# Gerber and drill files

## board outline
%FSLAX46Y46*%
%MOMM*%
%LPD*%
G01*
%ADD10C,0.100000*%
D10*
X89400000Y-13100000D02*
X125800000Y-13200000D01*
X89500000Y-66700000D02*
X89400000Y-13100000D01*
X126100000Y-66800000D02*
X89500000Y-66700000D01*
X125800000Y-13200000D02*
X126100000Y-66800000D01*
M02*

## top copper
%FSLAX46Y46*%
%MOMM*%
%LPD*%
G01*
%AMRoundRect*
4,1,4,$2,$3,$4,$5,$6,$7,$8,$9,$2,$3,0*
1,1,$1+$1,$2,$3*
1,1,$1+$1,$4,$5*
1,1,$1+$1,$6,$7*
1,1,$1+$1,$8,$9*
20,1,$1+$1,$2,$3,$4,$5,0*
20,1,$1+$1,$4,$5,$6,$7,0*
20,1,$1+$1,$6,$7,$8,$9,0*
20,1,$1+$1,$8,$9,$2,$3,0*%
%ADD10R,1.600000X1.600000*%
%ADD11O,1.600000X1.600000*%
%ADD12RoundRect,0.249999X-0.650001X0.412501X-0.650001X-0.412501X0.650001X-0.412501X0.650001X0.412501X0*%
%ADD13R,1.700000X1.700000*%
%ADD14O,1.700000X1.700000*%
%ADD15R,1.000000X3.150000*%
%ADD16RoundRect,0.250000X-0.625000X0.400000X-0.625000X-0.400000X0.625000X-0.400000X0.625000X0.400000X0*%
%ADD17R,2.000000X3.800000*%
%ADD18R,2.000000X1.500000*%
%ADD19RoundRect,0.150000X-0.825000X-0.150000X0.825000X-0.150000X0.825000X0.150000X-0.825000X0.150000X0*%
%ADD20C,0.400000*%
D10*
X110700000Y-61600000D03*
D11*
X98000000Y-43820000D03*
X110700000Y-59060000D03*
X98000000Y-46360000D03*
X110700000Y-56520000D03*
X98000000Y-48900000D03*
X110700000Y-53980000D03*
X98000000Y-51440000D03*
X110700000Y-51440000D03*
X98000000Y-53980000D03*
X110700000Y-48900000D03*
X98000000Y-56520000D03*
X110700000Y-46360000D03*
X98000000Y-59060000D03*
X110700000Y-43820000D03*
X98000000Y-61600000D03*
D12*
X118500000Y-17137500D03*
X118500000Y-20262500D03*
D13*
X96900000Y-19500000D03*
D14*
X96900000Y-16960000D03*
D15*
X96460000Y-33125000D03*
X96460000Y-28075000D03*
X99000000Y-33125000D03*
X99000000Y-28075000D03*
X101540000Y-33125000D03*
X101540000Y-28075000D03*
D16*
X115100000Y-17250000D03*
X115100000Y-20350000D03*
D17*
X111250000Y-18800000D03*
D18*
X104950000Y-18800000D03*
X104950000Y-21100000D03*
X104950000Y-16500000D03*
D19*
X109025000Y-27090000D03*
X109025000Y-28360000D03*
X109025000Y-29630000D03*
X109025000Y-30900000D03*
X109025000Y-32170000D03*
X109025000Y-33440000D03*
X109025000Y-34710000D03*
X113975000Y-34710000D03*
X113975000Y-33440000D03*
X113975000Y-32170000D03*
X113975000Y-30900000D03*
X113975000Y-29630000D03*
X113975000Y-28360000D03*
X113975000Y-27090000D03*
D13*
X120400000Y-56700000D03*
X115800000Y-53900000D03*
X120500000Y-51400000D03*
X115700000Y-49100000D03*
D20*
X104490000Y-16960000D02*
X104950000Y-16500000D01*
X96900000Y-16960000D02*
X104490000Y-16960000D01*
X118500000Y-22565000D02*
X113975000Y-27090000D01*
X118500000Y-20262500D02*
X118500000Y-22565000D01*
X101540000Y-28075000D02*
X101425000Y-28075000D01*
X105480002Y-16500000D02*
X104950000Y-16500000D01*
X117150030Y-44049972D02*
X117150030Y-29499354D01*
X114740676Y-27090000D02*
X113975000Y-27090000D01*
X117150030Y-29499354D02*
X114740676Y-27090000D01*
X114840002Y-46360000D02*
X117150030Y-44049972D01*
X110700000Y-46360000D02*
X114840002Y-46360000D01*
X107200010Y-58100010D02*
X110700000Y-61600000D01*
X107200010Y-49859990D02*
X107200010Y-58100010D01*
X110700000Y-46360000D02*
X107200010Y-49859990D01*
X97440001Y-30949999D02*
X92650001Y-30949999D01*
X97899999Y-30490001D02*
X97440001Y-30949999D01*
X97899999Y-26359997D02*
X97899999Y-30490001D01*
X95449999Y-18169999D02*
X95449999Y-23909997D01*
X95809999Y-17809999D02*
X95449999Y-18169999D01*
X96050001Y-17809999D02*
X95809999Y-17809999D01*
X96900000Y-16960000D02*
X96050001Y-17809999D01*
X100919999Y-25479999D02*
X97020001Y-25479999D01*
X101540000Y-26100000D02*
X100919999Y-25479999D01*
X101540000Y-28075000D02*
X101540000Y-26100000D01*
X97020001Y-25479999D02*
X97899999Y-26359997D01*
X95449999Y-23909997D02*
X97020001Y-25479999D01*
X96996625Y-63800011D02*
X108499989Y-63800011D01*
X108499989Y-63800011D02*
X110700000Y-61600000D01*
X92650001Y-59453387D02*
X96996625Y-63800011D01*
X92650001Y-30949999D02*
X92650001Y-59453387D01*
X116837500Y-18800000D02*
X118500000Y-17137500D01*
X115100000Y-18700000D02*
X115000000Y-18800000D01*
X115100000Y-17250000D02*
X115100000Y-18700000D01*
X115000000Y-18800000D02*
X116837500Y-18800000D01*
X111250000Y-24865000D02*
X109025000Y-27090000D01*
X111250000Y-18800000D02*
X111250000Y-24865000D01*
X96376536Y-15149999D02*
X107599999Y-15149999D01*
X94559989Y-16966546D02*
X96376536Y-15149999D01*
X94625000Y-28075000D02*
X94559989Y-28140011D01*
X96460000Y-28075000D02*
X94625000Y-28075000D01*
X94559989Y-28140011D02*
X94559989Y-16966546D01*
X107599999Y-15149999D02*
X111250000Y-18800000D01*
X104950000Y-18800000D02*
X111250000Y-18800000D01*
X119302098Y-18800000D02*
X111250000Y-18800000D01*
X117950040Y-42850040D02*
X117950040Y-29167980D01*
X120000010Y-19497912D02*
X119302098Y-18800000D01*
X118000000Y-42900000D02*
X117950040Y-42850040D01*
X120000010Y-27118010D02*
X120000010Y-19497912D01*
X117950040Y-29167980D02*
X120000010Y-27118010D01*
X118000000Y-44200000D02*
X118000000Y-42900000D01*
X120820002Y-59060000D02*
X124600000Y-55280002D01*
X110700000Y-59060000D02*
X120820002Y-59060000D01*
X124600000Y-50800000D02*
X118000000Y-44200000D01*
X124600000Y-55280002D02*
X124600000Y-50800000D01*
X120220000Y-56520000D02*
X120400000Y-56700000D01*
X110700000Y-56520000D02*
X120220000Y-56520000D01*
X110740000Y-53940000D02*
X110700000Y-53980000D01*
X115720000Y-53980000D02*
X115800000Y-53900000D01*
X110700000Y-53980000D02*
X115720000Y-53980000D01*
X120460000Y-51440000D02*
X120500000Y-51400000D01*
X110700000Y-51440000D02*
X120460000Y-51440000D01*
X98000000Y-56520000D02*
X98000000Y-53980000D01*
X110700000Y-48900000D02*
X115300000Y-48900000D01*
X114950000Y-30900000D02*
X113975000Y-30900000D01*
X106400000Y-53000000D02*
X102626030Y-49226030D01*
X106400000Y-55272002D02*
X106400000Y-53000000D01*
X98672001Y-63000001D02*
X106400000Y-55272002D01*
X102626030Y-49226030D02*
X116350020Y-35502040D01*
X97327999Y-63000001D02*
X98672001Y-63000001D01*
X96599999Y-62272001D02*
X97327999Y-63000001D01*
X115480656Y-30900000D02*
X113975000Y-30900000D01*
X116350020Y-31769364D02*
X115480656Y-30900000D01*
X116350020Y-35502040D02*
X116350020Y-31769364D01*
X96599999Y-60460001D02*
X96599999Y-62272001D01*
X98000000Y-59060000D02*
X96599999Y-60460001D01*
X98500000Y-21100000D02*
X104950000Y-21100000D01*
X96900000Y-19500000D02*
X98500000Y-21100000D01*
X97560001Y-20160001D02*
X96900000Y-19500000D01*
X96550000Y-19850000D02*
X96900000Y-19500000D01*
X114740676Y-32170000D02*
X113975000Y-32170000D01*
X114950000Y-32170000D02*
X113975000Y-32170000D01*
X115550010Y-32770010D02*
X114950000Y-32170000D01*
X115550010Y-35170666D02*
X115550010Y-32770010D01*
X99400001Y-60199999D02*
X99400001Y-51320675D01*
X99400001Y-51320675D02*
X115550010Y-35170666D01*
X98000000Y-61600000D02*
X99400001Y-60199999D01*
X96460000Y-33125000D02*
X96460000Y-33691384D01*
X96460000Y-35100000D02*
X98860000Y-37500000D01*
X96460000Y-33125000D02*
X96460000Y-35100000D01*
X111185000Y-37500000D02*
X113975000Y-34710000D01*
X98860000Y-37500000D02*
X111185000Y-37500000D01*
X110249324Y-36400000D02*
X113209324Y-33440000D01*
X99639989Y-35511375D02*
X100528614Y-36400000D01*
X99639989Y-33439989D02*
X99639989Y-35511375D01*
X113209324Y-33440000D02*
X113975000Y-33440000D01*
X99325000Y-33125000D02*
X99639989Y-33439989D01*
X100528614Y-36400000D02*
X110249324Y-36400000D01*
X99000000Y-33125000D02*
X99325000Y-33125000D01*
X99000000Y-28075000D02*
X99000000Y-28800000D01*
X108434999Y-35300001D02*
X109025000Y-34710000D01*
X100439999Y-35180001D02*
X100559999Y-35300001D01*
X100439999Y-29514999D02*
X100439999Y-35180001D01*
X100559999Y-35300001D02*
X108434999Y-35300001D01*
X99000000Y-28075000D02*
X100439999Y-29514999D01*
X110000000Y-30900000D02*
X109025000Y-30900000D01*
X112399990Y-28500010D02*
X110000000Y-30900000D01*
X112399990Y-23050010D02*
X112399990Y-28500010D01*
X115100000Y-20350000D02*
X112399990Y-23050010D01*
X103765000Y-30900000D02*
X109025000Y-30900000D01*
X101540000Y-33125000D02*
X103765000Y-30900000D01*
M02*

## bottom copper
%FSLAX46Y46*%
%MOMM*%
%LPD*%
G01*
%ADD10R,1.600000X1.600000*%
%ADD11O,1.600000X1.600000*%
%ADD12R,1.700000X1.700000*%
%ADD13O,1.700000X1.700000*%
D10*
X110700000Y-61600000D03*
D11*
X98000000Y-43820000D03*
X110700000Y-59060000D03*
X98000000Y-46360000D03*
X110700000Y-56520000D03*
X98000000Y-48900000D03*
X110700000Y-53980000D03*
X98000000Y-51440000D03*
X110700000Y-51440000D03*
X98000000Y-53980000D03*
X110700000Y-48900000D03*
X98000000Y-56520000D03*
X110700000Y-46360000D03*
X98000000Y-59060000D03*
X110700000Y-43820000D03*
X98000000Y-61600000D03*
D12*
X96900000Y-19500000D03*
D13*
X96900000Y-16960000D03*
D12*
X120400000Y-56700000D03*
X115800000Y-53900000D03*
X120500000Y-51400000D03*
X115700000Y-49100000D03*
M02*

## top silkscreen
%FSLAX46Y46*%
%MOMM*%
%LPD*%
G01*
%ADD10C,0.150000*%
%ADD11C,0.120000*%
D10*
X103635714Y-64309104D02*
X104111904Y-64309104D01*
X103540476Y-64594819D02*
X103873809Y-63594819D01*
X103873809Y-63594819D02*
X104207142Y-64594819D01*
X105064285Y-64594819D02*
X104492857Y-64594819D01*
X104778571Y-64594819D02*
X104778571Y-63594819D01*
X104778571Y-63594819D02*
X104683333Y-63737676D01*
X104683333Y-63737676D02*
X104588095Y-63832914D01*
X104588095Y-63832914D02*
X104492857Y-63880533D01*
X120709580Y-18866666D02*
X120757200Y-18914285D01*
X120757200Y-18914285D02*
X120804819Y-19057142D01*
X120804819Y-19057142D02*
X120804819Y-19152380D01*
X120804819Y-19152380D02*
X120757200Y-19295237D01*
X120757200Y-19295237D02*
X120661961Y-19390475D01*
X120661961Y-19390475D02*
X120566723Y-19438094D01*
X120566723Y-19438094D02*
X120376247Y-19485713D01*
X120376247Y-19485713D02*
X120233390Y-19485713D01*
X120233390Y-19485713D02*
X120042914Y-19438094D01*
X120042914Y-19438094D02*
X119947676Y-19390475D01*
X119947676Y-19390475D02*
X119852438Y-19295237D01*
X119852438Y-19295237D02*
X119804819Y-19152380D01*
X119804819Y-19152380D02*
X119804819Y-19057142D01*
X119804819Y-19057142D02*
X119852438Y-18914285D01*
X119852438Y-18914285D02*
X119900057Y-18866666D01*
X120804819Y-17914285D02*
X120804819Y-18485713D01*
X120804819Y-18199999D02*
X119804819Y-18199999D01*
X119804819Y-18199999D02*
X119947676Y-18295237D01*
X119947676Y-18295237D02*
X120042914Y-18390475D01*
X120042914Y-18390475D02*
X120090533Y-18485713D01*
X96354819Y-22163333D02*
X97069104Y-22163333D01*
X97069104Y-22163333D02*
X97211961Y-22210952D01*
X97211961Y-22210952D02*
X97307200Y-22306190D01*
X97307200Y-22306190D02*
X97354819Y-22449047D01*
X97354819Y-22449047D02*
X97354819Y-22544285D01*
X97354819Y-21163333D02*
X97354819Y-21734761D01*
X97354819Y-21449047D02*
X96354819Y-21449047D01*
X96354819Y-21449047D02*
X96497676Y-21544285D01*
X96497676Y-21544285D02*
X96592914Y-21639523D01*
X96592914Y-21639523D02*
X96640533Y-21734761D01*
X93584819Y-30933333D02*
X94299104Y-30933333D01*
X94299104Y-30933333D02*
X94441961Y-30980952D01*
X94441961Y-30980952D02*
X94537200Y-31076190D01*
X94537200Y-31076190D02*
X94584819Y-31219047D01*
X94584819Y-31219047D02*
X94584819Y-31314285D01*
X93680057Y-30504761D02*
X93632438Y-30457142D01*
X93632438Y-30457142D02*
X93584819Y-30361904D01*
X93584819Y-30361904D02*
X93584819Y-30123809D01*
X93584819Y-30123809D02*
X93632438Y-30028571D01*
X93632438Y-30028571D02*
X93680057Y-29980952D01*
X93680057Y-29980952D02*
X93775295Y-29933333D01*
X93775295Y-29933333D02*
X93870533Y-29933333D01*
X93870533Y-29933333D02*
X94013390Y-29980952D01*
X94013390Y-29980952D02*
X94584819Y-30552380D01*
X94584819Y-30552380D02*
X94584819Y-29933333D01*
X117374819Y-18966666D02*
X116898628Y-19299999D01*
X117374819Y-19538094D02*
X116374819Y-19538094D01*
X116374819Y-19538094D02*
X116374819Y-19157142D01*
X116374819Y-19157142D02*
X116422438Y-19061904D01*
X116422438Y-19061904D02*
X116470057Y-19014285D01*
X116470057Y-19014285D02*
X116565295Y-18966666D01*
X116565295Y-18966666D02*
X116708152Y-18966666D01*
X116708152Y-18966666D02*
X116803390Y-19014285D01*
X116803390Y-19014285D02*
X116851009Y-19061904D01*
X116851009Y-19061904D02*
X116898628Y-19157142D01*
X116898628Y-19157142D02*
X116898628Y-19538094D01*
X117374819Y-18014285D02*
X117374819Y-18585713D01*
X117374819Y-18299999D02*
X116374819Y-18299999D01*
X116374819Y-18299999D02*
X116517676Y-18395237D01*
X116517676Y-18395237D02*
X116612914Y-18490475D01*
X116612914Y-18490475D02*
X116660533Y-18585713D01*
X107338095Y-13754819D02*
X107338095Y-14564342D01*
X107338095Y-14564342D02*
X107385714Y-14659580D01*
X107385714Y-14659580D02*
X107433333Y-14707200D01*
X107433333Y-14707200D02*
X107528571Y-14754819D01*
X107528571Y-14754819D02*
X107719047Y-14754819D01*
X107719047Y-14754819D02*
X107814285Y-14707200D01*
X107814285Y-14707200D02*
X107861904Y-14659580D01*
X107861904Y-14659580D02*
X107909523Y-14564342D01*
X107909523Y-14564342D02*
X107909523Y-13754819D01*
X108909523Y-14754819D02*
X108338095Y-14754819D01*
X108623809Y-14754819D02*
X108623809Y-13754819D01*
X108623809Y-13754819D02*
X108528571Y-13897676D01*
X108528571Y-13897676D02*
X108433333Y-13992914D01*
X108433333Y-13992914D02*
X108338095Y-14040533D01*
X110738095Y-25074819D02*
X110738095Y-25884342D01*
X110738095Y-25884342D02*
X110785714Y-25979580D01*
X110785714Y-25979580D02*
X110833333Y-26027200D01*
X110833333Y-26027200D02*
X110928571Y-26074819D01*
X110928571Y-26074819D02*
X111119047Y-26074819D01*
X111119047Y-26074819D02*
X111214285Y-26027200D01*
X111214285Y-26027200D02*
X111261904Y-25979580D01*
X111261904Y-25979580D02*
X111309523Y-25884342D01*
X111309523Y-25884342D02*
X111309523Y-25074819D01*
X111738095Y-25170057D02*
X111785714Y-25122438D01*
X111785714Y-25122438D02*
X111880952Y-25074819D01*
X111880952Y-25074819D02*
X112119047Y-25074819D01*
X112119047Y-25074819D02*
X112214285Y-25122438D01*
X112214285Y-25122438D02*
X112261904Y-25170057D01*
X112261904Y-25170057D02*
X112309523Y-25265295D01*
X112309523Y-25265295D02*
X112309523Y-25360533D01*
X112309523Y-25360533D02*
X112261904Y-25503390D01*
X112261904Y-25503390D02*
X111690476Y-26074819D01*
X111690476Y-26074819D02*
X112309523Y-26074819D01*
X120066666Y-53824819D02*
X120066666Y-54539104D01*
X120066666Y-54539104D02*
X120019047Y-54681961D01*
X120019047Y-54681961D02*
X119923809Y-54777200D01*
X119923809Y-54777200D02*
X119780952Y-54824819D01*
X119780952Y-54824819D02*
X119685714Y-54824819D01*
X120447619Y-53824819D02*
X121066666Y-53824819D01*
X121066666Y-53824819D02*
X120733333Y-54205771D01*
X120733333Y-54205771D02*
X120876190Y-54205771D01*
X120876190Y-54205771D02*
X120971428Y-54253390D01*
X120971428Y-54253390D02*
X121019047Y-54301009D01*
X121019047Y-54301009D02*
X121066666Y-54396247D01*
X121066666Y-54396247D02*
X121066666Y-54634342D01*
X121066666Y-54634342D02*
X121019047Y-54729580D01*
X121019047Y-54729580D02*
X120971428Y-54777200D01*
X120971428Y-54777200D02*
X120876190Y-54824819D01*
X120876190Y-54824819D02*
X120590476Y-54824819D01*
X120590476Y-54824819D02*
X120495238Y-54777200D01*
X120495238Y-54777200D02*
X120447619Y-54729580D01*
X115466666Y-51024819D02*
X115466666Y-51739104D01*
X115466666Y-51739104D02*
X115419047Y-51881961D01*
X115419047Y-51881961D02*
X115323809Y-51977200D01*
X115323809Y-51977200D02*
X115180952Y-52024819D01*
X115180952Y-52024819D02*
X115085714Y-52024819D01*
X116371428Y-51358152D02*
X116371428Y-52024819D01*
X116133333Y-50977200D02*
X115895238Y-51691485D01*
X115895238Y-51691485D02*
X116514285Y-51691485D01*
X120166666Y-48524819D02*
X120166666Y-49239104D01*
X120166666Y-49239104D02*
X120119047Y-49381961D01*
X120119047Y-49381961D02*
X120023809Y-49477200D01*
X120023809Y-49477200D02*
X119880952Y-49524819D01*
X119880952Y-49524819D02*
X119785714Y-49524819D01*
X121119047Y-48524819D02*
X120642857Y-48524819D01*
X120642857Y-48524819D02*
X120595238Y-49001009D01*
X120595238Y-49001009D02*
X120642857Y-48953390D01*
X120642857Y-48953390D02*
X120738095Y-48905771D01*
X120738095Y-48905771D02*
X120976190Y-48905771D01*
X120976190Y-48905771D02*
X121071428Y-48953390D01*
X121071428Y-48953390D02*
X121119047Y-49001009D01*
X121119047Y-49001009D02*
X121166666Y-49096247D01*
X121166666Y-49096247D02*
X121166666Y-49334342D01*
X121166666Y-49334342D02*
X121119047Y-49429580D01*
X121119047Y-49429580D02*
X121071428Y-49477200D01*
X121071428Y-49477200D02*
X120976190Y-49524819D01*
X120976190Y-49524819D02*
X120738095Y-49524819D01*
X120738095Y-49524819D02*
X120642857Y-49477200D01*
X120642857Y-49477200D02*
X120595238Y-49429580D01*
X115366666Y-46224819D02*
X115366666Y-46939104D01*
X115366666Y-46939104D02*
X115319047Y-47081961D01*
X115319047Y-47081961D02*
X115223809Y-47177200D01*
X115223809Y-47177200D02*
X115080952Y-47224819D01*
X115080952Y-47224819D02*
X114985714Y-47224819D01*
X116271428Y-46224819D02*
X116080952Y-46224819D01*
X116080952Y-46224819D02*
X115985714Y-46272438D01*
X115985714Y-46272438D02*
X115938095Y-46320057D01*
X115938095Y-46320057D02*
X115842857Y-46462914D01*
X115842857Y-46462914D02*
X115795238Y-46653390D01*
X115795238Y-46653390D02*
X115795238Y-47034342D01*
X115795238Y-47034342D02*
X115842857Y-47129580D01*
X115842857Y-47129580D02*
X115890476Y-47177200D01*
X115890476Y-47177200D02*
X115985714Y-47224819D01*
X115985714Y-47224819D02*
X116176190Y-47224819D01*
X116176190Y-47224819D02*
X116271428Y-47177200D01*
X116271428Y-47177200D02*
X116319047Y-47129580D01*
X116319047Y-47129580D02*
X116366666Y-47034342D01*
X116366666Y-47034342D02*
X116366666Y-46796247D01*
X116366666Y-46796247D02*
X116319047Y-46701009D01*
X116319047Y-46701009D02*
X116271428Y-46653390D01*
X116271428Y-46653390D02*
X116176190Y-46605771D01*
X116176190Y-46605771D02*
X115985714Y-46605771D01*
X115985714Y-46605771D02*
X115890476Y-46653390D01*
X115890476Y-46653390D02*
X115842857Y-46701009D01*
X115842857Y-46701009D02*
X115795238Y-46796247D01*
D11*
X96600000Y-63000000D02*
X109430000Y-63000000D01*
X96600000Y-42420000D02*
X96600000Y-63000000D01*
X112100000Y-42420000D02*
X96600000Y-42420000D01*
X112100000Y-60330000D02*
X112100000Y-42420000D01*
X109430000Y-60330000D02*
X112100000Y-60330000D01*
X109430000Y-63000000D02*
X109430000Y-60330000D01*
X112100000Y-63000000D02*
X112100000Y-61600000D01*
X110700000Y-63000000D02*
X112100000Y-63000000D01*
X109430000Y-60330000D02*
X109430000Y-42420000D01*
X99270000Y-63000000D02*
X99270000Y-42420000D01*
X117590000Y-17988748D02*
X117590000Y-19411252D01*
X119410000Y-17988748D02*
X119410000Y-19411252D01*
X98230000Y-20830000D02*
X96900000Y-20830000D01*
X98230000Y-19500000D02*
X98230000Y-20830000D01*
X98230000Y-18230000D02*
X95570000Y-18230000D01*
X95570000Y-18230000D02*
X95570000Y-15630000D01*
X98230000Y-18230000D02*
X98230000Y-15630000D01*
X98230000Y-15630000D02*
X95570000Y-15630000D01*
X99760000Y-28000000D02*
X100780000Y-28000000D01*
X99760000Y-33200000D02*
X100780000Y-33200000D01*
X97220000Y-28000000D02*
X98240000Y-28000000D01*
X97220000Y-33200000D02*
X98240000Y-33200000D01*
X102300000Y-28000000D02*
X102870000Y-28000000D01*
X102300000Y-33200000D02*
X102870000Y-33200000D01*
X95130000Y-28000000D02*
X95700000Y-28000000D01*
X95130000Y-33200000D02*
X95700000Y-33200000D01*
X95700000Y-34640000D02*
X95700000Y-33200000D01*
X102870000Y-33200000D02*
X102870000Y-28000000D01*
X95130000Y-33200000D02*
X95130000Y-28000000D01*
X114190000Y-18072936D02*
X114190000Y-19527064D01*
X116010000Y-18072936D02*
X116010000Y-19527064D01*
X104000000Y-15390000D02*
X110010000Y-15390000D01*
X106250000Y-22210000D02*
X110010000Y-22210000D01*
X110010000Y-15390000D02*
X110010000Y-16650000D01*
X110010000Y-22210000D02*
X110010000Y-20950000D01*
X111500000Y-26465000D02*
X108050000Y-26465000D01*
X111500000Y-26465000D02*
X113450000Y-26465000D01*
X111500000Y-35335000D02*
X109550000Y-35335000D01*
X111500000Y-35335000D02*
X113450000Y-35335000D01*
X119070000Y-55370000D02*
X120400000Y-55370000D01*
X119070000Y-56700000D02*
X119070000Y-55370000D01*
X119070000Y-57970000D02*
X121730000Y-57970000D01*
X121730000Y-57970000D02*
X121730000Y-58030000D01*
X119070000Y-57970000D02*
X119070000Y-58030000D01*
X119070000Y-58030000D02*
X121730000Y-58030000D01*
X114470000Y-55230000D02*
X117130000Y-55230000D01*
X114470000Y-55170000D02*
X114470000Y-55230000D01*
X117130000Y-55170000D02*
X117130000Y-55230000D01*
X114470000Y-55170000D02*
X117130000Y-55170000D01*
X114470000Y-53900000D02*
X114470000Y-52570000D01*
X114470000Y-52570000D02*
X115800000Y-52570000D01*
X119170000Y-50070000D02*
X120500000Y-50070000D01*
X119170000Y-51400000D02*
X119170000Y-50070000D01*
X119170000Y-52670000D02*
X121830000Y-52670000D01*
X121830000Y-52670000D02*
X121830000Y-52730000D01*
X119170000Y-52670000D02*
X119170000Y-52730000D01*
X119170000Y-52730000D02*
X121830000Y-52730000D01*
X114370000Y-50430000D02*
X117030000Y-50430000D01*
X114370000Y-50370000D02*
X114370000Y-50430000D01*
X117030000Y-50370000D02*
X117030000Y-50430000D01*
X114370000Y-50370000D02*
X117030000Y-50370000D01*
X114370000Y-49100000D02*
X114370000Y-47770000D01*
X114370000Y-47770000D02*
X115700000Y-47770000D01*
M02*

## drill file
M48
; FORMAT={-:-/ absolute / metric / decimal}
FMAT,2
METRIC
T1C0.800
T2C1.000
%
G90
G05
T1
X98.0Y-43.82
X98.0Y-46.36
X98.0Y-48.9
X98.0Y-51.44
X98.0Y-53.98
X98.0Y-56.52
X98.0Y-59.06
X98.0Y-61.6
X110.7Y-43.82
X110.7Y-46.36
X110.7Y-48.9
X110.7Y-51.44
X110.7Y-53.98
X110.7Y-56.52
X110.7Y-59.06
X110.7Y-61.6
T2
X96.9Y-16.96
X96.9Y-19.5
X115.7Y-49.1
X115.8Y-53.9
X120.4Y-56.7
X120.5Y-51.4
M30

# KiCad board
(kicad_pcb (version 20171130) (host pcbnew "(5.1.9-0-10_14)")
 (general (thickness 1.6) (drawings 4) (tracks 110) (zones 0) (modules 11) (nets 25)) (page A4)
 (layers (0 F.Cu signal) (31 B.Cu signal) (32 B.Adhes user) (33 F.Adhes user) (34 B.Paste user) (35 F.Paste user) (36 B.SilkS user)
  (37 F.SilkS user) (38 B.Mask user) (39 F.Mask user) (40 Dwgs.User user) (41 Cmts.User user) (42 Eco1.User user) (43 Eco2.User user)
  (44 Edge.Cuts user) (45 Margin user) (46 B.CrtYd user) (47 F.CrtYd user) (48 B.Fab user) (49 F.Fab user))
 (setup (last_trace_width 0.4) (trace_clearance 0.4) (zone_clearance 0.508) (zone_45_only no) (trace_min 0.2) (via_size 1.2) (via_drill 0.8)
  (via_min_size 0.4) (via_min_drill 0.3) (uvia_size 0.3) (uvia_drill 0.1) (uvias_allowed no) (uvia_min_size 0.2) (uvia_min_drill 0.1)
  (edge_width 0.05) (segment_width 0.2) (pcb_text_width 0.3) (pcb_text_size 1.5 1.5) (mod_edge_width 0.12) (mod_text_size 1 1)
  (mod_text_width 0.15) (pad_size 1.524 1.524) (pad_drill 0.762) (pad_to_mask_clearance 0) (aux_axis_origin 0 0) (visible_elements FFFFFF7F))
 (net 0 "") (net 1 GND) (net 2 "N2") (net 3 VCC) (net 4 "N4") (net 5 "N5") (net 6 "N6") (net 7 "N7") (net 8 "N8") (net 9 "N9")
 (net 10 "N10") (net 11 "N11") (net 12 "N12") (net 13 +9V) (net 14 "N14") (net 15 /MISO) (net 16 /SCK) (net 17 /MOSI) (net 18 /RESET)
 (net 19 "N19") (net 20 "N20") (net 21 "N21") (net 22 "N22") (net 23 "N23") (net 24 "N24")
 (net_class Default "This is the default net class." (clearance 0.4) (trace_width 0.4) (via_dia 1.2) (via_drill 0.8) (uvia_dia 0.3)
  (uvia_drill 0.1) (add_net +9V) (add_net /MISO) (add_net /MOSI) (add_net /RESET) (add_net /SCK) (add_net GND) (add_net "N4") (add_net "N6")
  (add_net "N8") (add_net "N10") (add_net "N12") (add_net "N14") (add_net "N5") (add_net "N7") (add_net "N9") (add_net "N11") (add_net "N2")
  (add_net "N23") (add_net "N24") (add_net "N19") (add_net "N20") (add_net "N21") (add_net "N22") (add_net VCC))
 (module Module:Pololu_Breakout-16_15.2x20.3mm (layer F.Cu) (at 110.7 61.6 180)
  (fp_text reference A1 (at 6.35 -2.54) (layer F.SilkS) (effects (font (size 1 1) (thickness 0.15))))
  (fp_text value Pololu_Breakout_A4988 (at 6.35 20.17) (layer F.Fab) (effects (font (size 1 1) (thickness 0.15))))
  (fp_line (start 14.1 -1.4) (end 1.27 -1.4) (layer F.SilkS) (width 0.12))
  (fp_line (start 14.1 19.18) (end 14.1 -1.4) (layer F.SilkS) (width 0.12))
  (fp_line (start -1.4 19.18) (end 14.1 19.18) (layer F.SilkS) (width 0.12))
  (fp_line (start -1.4 1.27) (end -1.4 19.18) (layer F.SilkS) (width 0.12))
  (fp_line (start 1.27 1.27) (end -1.4 1.27) (layer F.SilkS) (width 0.12))
  (fp_line (start 1.27 -1.4) (end 1.27 1.27) (layer F.SilkS) (width 0.12))
  (fp_line (start -1.4 -1.4) (end -1.4 0) (layer F.SilkS) (width 0.12))
  (fp_line (start 0 -1.4) (end -1.4 -1.4) (layer F.SilkS) (width 0.12))
  (fp_line (start 1.27 1.27) (end 1.27 19.18) (layer F.SilkS) (width 0.12))
  (fp_line (start 11.43 -1.4) (end 11.43 19.18) (layer F.SilkS) (width 0.12))
  (pad 1 thru_hole rect (at 0 0 180) (size 1.6 1.6) (drill 0.8) (layers *.Cu *.Mask) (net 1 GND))
  (pad 9 thru_hole oval (at 12.7 17.78 180) (size 1.6 1.6) (drill 0.8) (layers *.Cu *.Mask) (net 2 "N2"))
  (pad 2 thru_hole oval (at 0 2.54 180) (size 1.6 1.6) (drill 0.8) (layers *.Cu *.Mask) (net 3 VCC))
  (pad 10 thru_hole oval (at 12.7 15.24 180) (size 1.6 1.6) (drill 0.8) (layers *.Cu *.Mask) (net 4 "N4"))
  (pad 3 thru_hole oval (at 0 5.08 180) (size 1.6 1.6) (drill 0.8) (layers *.Cu *.Mask) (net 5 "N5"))
  (pad 11 thru_hole oval (at 12.7 12.7 180) (size 1.6 1.6) (drill 0.8) (layers *.Cu *.Mask) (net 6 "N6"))
  (pad 4 thru_hole oval (at 0 7.62 180) (size 1.6 1.6) (drill 0.8) (layers *.Cu *.Mask) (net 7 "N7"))
  (pad 12 thru_hole oval (at 12.7 10.16 180) (size 1.6 1.6) (drill 0.8) (layers *.Cu *.Mask) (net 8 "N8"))
  (pad 5 thru_hole oval (at 0 10.16 180) (size 1.6 1.6) (drill 0.8) (layers *.Cu *.Mask) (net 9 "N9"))
  (pad 13 thru_hole oval (at 12.7 7.62 180) (size 1.6 1.6) (drill 0.8) (layers *.Cu *.Mask) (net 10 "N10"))
  (pad 6 thru_hole oval (at 0 12.7 180) (size 1.6 1.6) (drill 0.8) (layers *.Cu *.Mask) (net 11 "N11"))
  (pad 14 thru_hole oval (at 12.7 5.08 180) (size 1.6 1.6) (drill 0.8) (layers *.Cu *.Mask) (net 10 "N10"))
  (pad 7 thru_hole oval (at 0 15.24 180) (size 1.6 1.6) (drill 0.8) (layers *.Cu *.Mask) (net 1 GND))
  (pad 15 thru_hole oval (at 12.7 2.54 180) (size 1.6 1.6) (drill 0.8) (layers *.Cu *.Mask) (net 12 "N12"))
  (pad 8 thru_hole oval (at 0 17.78 180) (size 1.6 1.6) (drill 0.8) (layers *.Cu *.Mask) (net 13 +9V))
  (pad 16 thru_hole oval (at 12.7 0 180) (size 1.6 1.6) (drill 0.8) (layers *.Cu *.Mask) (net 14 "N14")))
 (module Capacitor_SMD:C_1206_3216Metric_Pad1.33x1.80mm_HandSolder (layer F.Cu) (at 118.5 18.7 270)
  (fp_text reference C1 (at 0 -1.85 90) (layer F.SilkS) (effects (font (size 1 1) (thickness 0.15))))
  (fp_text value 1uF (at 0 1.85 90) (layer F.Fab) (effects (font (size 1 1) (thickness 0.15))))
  (fp_line (start -0.711252 0.91) (end 0.711252 0.91) (layer F.SilkS) (width 0.12))
  (fp_line (start -0.711252 -0.91) (end 0.711252 -0.91) (layer F.SilkS) (width 0.12))
  (pad 1 smd roundrect (at -1.5625 0 270) (size 1.325 1.8) (layers F.Cu F.Paste F.Mask) (roundrect_rratio 0.1886784905660377) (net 3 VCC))
  (pad 2 smd roundrect (at 1.5625 0 270) (size 1.325 1.8) (layers F.Cu F.Paste F.Mask) (roundrect_rratio 0.1886784905660377) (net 1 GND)))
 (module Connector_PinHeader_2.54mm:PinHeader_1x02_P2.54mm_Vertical (layer F.Cu) (at 96.9 19.5 180)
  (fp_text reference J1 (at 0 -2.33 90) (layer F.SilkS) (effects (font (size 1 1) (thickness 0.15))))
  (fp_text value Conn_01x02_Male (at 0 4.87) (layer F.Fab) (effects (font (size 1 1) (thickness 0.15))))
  (fp_line (start -1.33 -1.33) (end 0 -1.33) (layer F.SilkS) (width 0.12))
  (fp_line (start -1.33 0) (end -1.33 -1.33) (layer F.SilkS) (width 0.12))
  (fp_line (start -1.33 1.27) (end 1.33 1.27) (layer F.SilkS) (width 0.12))
  (fp_line (start 1.33 1.27) (end 1.33 3.87) (layer F.SilkS) (width 0.12))
  (fp_line (start -1.33 1.27) (end -1.33 3.87) (layer F.SilkS) (width 0.12))
  (fp_line (start -1.33 3.87) (end 1.33 3.87) (layer F.SilkS) (width 0.12))
  (pad 1 thru_hole rect (at 0 0 180) (size 1.7 1.7) (drill 1) (layers *.Cu *.Mask) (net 13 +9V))
  (pad 2 thru_hole oval (at 0 2.54 180) (size 1.7 1.7) (drill 1) (layers *.Cu *.Mask) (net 1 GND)))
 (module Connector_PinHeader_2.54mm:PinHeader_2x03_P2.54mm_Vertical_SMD (layer F.Cu) (at 99 30.6 90)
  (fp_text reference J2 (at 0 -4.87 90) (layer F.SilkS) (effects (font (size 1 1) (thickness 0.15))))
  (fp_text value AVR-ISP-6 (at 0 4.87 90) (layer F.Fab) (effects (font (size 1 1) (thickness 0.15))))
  (fp_line (start 2.6 0.76) (end 2.6 1.78) (layer F.SilkS) (width 0.12))
  (fp_line (start -2.6 0.76) (end -2.6 1.78) (layer F.SilkS) (width 0.12))
  (fp_line (start 2.6 -1.78) (end 2.6 -0.76) (layer F.SilkS) (width 0.12))
  (fp_line (start -2.6 -1.78) (end -2.6 -0.76) (layer F.SilkS) (width 0.12))
  (fp_line (start 2.6 3.3) (end 2.6 3.87) (layer F.SilkS) (width 0.12))
  (fp_line (start -2.6 3.3) (end -2.6 3.87) (layer F.SilkS) (width 0.12))
  (fp_line (start 2.6 -3.87) (end 2.6 -3.3) (layer F.SilkS) (width 0.12))
  (fp_line (start -2.6 -3.87) (end -2.6 -3.3) (layer F.SilkS) (width 0.12))
  (fp_line (start -4.04 -3.3) (end -2.6 -3.3) (layer F.SilkS) (width 0.12))
  (fp_line (start -2.6 3.87) (end 2.6 3.87) (layer F.SilkS) (width 0.12))
  (fp_line (start -2.6 -3.87) (end 2.6 -3.87) (layer F.SilkS) (width 0.12))
  (pad 1 smd rect (at -2.525 -2.54 90) (size 3.15 1) (layers F.Cu F.Paste F.Mask) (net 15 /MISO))
  (pad 2 smd rect (at 2.525 -2.54 90) (size 3.15 1) (layers F.Cu F.Paste F.Mask) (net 3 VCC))
  (pad 3 smd rect (at -2.525 0 90) (size 3.15 1) (layers F.Cu F.Paste F.Mask) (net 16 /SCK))
  (pad 4 smd rect (at 2.525 0 90) (size 3.15 1) (layers F.Cu F.Paste F.Mask) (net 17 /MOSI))
  (pad 5 smd rect (at -2.525 2.54 90) (size 3.15 1) (layers F.Cu F.Paste F.Mask) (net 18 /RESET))
  (pad 6 smd rect (at 2.525 2.54 90) (size 3.15 1) (layers F.Cu F.Paste F.Mask) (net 1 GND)))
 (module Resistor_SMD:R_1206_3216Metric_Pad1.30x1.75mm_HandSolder (layer F.Cu) (at 115.1 18.8 270)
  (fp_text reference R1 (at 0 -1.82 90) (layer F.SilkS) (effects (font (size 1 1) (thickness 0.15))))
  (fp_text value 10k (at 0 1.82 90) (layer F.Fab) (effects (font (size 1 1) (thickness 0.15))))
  (fp_line (start -0.727064 0.91) (end 0.727064 0.91) (layer F.SilkS) (width 0.12))
  (fp_line (start -0.727064 -0.91) (end 0.727064 -0.91) (layer F.SilkS) (width 0.12))
  (pad 1 smd roundrect (at -1.55 0 270) (size 1.3 1.75) (layers F.Cu F.Paste F.Mask) (roundrect_rratio 0.1923076923076923) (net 3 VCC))
  (pad 2 smd roundrect (at 1.55 0 270) (size 1.3 1.75) (layers F.Cu F.Paste F.Mask) (roundrect_rratio 0.1923076923076923) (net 18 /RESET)))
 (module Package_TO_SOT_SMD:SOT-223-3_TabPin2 (layer F.Cu) (at 108.1 18.8)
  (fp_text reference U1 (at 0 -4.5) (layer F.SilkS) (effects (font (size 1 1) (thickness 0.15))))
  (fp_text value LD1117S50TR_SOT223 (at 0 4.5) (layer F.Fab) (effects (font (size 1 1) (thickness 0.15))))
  (fp_line (start -4.1 -3.41) (end 1.91 -3.41) (layer F.SilkS) (width 0.12))
  (fp_line (start -1.85 3.41) (end 1.91 3.41) (layer F.SilkS) (width 0.12))
  (fp_line (start 1.91 -3.41) (end 1.91 -2.15) (layer F.SilkS) (width 0.12))
  (fp_line (start 1.91 3.41) (end 1.91 2.15) (layer F.SilkS) (width 0.12))
  (pad 2 smd rect (at 3.15 0) (size 2 3.8) (layers F.Cu F.Paste F.Mask) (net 3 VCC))
  (pad 2 smd rect (at -3.15 0) (size 2 1.5) (layers F.Cu F.Paste F.Mask) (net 3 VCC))
  (pad 3 smd rect (at -3.15 2.3) (size 2 1.5) (layers F.Cu F.Paste F.Mask) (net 13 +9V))
  (pad 1 smd rect (at -3.15 -2.3) (size 2 1.5) (layers F.Cu F.Paste F.Mask) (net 1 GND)))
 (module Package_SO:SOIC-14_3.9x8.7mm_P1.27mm (layer F.Cu) (at 111.5 30.9)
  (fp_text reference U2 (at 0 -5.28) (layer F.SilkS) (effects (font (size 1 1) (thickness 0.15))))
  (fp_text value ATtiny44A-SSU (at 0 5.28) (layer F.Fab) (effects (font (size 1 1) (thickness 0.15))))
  (fp_line (start 0 -4.435) (end -3.45 -4.435) (layer F.SilkS) (width 0.12))
  (fp_line (start 0 -4.435) (end 1.95 -4.435) (layer F.SilkS) (width 0.12))
  (fp_line (start 0 4.435) (end -1.95 4.435) (layer F.SilkS) (width 0.12))
  (fp_line (start 0 4.435) (end 1.95 4.435) (layer F.SilkS) (width 0.12))
  (pad 1 smd roundrect (at -2.475 -3.81) (size 1.95 0.6) (layers F.Cu F.Paste F.Mask) (roundrect_rratio 0.25) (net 3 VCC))
  (pad 2 smd roundrect (at -2.475 -2.54) (size 1.95 0.6) (layers F.Cu F.Paste F.Mask) (roundrect_rratio 0.25) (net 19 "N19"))
  (pad 3 smd roundrect (at -2.475 -1.27) (size 1.95 0.6) (layers F.Cu F.Paste F.Mask) (roundrect_rratio 0.25) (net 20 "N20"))
  (pad 4 smd roundrect (at -2.475 0) (size 1.95 0.6) (layers F.Cu F.Paste F.Mask) (roundrect_rratio 0.25) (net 18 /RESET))
  (pad 5 smd roundrect (at -2.475 1.27) (size 1.95 0.6) (layers F.Cu F.Paste F.Mask) (roundrect_rratio 0.25) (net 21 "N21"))
  (pad 6 smd roundrect (at -2.475 2.54) (size 1.95 0.6) (layers F.Cu F.Paste F.Mask) (roundrect_rratio 0.25) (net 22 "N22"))
  (pad 7 smd roundrect (at -2.475 3.81) (size 1.95 0.6) (layers F.Cu F.Paste F.Mask) (roundrect_rratio 0.25) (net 17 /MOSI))
  (pad 8 smd roundrect (at 2.475 3.81) (size 1.95 0.6) (layers F.Cu F.Paste F.Mask) (roundrect_rratio 0.25) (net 15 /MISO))
  (pad 9 smd roundrect (at 2.475 2.54) (size 1.95 0.6) (layers F.Cu F.Paste F.Mask) (roundrect_rratio 0.25) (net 16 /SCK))
  (pad 10 smd roundrect (at 2.475 1.27) (size 1.95 0.6) (layers F.Cu F.Paste F.Mask) (roundrect_rratio 0.25) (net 14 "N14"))
  (pad 11 smd roundrect (at 2.475 0) (size 1.95 0.6) (layers F.Cu F.Paste F.Mask) (roundrect_rratio 0.25) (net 12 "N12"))
  (pad 12 smd roundrect (at 2.475 -1.27) (size 1.95 0.6) (layers F.Cu F.Paste F.Mask) (roundrect_rratio 0.25) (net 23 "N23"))
  (pad 13 smd roundrect (at 2.475 -2.54) (size 1.95 0.6) (layers F.Cu F.Paste F.Mask) (roundrect_rratio 0.25) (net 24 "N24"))
  (pad 14 smd roundrect (at 2.475 -3.81) (size 1.95 0.6) (layers F.Cu F.Paste F.Mask) (roundrect_rratio 0.25) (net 1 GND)))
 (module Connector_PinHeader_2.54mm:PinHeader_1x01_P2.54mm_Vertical (layer F.Cu) (at 120.4 56.7)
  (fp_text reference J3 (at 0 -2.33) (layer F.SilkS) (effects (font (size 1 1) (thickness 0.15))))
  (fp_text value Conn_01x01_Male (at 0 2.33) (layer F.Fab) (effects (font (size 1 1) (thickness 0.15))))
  (fp_line (start -1.33 -1.33) (end 0 -1.33) (layer F.SilkS) (width 0.12))
  (fp_line (start -1.33 0) (end -1.33 -1.33) (layer F.SilkS) (width 0.12))
  (fp_line (start -1.33 1.27) (end 1.33 1.27) (layer F.SilkS) (width 0.12))
  (fp_line (start 1.33 1.27) (end 1.33 1.33) (layer F.SilkS) (width 0.12))
  (fp_line (start -1.33 1.27) (end -1.33 1.33) (layer F.SilkS) (width 0.12))
  (fp_line (start -1.33 1.33) (end 1.33 1.33) (layer F.SilkS) (width 0.12))
  (pad 1 thru_hole rect (at 0 0) (size 1.7 1.7) (drill 1) (layers *.Cu *.Mask) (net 5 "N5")))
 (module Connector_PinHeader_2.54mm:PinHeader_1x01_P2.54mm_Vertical (layer F.Cu) (at 115.8 53.9)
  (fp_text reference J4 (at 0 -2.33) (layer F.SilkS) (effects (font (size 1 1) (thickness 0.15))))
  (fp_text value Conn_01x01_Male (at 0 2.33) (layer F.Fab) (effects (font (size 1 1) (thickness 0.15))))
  (fp_line (start -1.33 1.33) (end 1.33 1.33) (layer F.SilkS) (width 0.12))
  (fp_line (start -1.33 1.27) (end -1.33 1.33) (layer F.SilkS) (width 0.12))
  (fp_line (start 1.33 1.27) (end 1.33 1.33) (layer F.SilkS) (width 0.12))
  (fp_line (start -1.33 1.27) (end 1.33 1.27) (layer F.SilkS) (width 0.12))
  (fp_line (start -1.33 0) (end -1.33 -1.33) (layer F.SilkS) (width 0.12))
  (fp_line (start -1.33 -1.33) (end 0 -1.33) (layer F.SilkS) (width 0.12))
  (pad 1 thru_hole rect (at 0 0) (size 1.7 1.7) (drill 1) (layers *.Cu *.Mask) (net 7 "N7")))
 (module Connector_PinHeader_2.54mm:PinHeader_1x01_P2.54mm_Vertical (layer F.Cu) (at 120.5 51.4)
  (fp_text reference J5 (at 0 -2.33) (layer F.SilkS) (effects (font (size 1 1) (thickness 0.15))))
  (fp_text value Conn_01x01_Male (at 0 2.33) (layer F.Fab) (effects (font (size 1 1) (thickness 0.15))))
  (fp_line (start -1.33 -1.33) (end 0 -1.33) (layer F.SilkS) (width 0.12))
  (fp_line (start -1.33 0) (end -1.33 -1.33) (layer F.SilkS) (width 0.12))
  (fp_line (start -1.33 1.27) (end 1.33 1.27) (layer F.SilkS) (width 0.12))
  (fp_line (start 1.33 1.27) (end 1.33 1.33) (layer F.SilkS) (width 0.12))
  (fp_line (start -1.33 1.27) (end -1.33 1.33) (layer F.SilkS) (width 0.12))
  (fp_line (start -1.33 1.33) (end 1.33 1.33) (layer F.SilkS) (width 0.12))
  (pad 1 thru_hole rect (at 0 0) (size 1.7 1.7) (drill 1) (layers *.Cu *.Mask) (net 9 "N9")))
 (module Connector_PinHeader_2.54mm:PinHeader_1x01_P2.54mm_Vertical (layer F.Cu) (at 115.7 49.1)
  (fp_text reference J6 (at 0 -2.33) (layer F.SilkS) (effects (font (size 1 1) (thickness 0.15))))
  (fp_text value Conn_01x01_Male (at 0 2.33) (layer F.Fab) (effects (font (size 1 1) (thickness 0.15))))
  (fp_line (start -1.33 1.33) (end 1.33 1.33) (layer F.SilkS) (width 0.12))
  (fp_line (start -1.33 1.27) (end -1.33 1.33) (layer F.SilkS) (width 0.12))
  (fp_line (start 1.33 1.27) (end 1.33 1.33) (layer F.SilkS) (width 0.12))
  (fp_line (start -1.33 1.27) (end 1.33 1.27) (layer F.SilkS) (width 0.12))
  (fp_line (start -1.33 0) (end -1.33 -1.33) (layer F.SilkS) (width 0.12))
  (fp_line (start -1.33 -1.33) (end 0 -1.33) (layer F.SilkS) (width 0.12))
  (pad 1 thru_hole rect (at 0 0) (size 1.7 1.7) (drill 1) (layers *.Cu *.Mask) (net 11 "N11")))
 (gr_line (start 89.4 13.1) (end 125.8 13.2) (layer Edge.Cuts) (width 0.1))
 (gr_line (start 89.5 66.7) (end 89.4 13.1) (layer Edge.Cuts) (width 0.1))
 (gr_line (start 126.1 66.8) (end 89.5 66.7) (layer Edge.Cuts) (width 0.1))
 (gr_line (start 125.8 13.2) (end 126.1 66.8) (layer Edge.Cuts) (width 0.1))
 (segment (start 104.49 16.96) (end 104.95 16.5) (width 0.4) (layer F.Cu) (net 1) (status 30))
 (segment (start 96.9 16.96) (end 104.49 16.96) (width 0.4) (layer F.Cu) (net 1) (status 30))
 (segment (start 118.5 22.565) (end 113.975 27.09) (width 0.4) (layer F.Cu) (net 1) (status 20))
 (segment (start 118.5 20.2625) (end 118.5 22.565) (width 0.4) (layer F.Cu) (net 1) (status 10))
 (segment (start 101.54 28.075) (end 101.425 28.075) (width 0.4) (layer F.Cu) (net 1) (status 30))
 (segment (start 105.480002 16.5) (end 104.95 16.5) (width 0.4) (layer F.Cu) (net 1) (status 30))
 (segment (start 117.15003 44.049972) (end 117.15003 29.499354) (width 0.4) (layer F.Cu) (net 1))
 (segment (start 114.740676 27.09) (end 113.975 27.09) (width 0.4) (layer F.Cu) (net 1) (status 30))
 (segment (start 117.15003 29.499354) (end 114.740676 27.09) (width 0.4) (layer F.Cu) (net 1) (status 20))
 (segment (start 114.840002 46.36) (end 117.15003 44.049972) (width 0.4) (layer F.Cu) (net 1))
 (segment (start 110.7 46.36) (end 114.840002 46.36) (width 0.4) (layer F.Cu) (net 1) (status 10))
 (segment (start 107.20001 58.10001) (end 110.7 61.6) (width 0.4) (layer F.Cu) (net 1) (status 20))
 (segment (start 107.20001 49.85999) (end 107.20001 58.10001) (width 0.4) (layer F.Cu) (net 1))
 (segment (start 110.7 46.36) (end 107.20001 49.85999) (width 0.4) (layer F.Cu) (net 1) (status 10))
 (segment (start 97.440001 30.949999) (end 92.650001 30.949999) (width 0.4) (layer F.Cu) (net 1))
 (segment (start 97.899999 30.490001) (end 97.440001 30.949999) (width 0.4) (layer F.Cu) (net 1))
 (segment (start 97.899999 26.359997) (end 97.899999 30.490001) (width 0.4) (layer F.Cu) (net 1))
 (segment (start 95.449999 18.169999) (end 95.449999 23.909997) (width 0.4) (layer F.Cu) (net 1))
 (segment (start 95.809999 17.809999) (end 95.449999 18.169999) (width 0.4) (layer F.Cu) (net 1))
 (segment (start 96.050001 17.809999) (end 95.809999 17.809999) (width 0.4) (layer F.Cu) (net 1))
 (segment (start 96.9 16.96) (end 96.050001 17.809999) (width 0.4) (layer F.Cu) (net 1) (status 10))
 (segment (start 100.919999 25.479999) (end 97.020001 25.479999) (width 0.4) (layer F.Cu) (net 1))
 (segment (start 101.54 26.1) (end 100.919999 25.479999) (width 0.4) (layer F.Cu) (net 1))
 (segment (start 101.54 28.075) (end 101.54 26.1) (width 0.4) (layer F.Cu) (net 1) (status 10))
 (segment (start 97.020001 25.479999) (end 97.899999 26.359997) (width 0.4) (layer F.Cu) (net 1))
 (segment (start 95.449999 23.909997) (end 97.020001 25.479999) (width 0.4) (layer F.Cu) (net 1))
 (segment (start 96.996625 63.800011) (end 108.499989 63.800011) (width 0.4) (layer F.Cu) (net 1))
 (segment (start 108.499989 63.800011) (end 110.7 61.6) (width 0.4) (layer F.Cu) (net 1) (status 20))
 (segment (start 92.650001 59.453387) (end 96.996625 63.800011) (width 0.4) (layer F.Cu) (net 1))
 (segment (start 92.650001 30.949999) (end 92.650001 59.453387) (width 0.4) (layer F.Cu) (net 1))
 (segment (start 116.8375 18.8) (end 118.5 17.1375) (width 0.4) (layer F.Cu) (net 3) (status 20))
 (segment (start 115.1 18.7) (end 115 18.8) (width 0.4) (layer F.Cu) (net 3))
 (segment (start 115.1 17.25) (end 115.1 18.7) (width 0.4) (layer F.Cu) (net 3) (status 10))
 (segment (start 115 18.8) (end 116.8375 18.8) (width 0.4) (layer F.Cu) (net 3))
 (segment (start 111.25 24.865) (end 109.025 27.09) (width 0.4) (layer F.Cu) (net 3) (status 20))
 (segment (start 111.25 18.8) (end 111.25 24.865) (width 0.4) (layer F.Cu) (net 3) (status 10))
 (segment (start 96.376536 15.149999) (end 107.599999 15.149999) (width 0.4) (layer F.Cu) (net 3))
 (segment (start 94.559989 16.966546) (end 96.376536 15.149999) (width 0.4) (layer F.Cu) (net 3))
 (segment (start 94.625 28.075) (end 94.559989 28.140011) (width 0.4) (layer F.Cu) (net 3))
 (segment (start 96.46 28.075) (end 94.625 28.075) (width 0.4) (layer F.Cu) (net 3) (status 10))
 (segment (start 94.559989 28.140011) (end 94.559989 16.966546) (width 0.4) (layer F.Cu) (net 3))
 (segment (start 107.599999 15.149999) (end 111.25 18.8) (width 0.4) (layer F.Cu) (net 3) (status 20))
 (segment (start 104.95 18.8) (end 111.25 18.8) (width 0.4) (layer F.Cu) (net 3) (status 30))
 (segment (start 119.302098 18.8) (end 111.25 18.8) (width 0.4) (layer F.Cu) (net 3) (status 20))
 (segment (start 117.95004 42.85004) (end 117.95004 29.16798) (width 0.4) (layer F.Cu) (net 3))
 (segment (start 120.00001 19.497912) (end 119.302098 18.8) (width 0.4) (layer F.Cu) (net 3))
 (segment (start 118 42.9) (end 117.95004 42.85004) (width 0.4) (layer F.Cu) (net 3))
 (segment (start 120.00001 27.11801) (end 120.00001 19.497912) (width 0.4) (layer F.Cu) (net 3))
 (segment (start 117.95004 29.16798) (end 120.00001 27.11801) (width 0.4) (layer F.Cu) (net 3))
 (segment (start 118 44.2) (end 118 42.9) (width 0.4) (layer F.Cu) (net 3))
 (segment (start 120.820002 59.06) (end 124.6 55.280002) (width 0.4) (layer F.Cu) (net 3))
 (segment (start 110.7 59.06) (end 120.820002 59.06) (width 0.4) (layer F.Cu) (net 3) (status 10))
 (segment (start 124.6 50.8) (end 118 44.2) (width 0.4) (layer F.Cu) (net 3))
 (segment (start 124.6 55.280002) (end 124.6 50.8) (width 0.4) (layer F.Cu) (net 3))
 (segment (start 120.22 56.52) (end 120.4 56.7) (width 0.4) (layer F.Cu) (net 5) (status 30))
 (segment (start 110.7 56.52) (end 120.22 56.52) (width 0.4) (layer F.Cu) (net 5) (status 30))
 (segment (start 110.74 53.94) (end 110.7 53.98) (width 0.4) (layer F.Cu) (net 7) (status 30))
 (segment (start 115.72 53.98) (end 115.8 53.9) (width 0.4) (layer F.Cu) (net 7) (status 30))
 (segment (start 110.7 53.98) (end 115.72 53.98) (width 0.4) (layer F.Cu) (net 7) (status 30))
 (segment (start 120.46 51.44) (end 120.5 51.4) (width 0.4) (layer F.Cu) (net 9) (status 30))
 (segment (start 110.7 51.44) (end 120.46 51.44) (width 0.4) (layer F.Cu) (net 9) (status 30))
 (segment (start 98 56.52) (end 98 53.98) (width 0.4) (layer F.Cu) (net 10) (status 30))
 (segment (start 110.7 48.9) (end 115.3 48.9) (width 0.4) (layer F.Cu) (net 11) (status 30))
 (segment (start 114.95 30.9) (end 113.975 30.9) (width 0.4) (layer F.Cu) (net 12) (status 20))
 (segment (start 106.4 53) (end 102.62603 49.22603) (width 0.4) (layer F.Cu) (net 12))
 (segment (start 106.4 55.272002) (end 106.4 53) (width 0.4) (layer F.Cu) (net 12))
 (segment (start 98.672001 63.000001) (end 106.4 55.272002) (width 0.4) (layer F.Cu) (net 12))
 (segment (start 102.62603 49.22603) (end 116.35002 35.50204) (width 0.4) (layer F.Cu) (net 12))
 (segment (start 97.327999 63.000001) (end 98.672001 63.000001) (width 0.4) (layer F.Cu) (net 12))
 (segment (start 96.599999 62.272001) (end 97.327999 63.000001) (width 0.4) (layer F.Cu) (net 12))
 (segment (start 115.480656 30.9) (end 113.975 30.9) (width 0.4) (layer F.Cu) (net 12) (status 20))
 (segment (start 116.35002 31.769364) (end 115.480656 30.9) (width 0.4) (layer F.Cu) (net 12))
 (segment (start 116.35002 35.50204) (end 116.35002 31.769364) (width 0.4) (layer F.Cu) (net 12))
 (segment (start 96.599999 60.460001) (end 96.599999 62.272001) (width 0.4) (layer F.Cu) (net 12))
 (segment (start 98 59.06) (end 96.599999 60.460001) (width 0.4) (layer F.Cu) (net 12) (status 10))
 (segment (start 98.5 21.1) (end 104.95 21.1) (width 0.4) (layer F.Cu) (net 13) (status 20))
 (segment (start 96.9 19.5) (end 98.5 21.1) (width 0.4) (layer F.Cu) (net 13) (status 10))
 (segment (start 97.560001 20.160001) (end 96.9 19.5) (width 0.4) (layer F.Cu) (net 13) (status 30))
 (segment (start 96.55 19.85) (end 96.9 19.5) (width 0.4) (layer F.Cu) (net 13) (status 30))
 (segment (start 114.740676 32.17) (end 113.975 32.17) (width 0.4) (layer F.Cu) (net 14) (status 30))
 (segment (start 114.95 32.17) (end 113.975 32.17) (width 0.4) (layer F.Cu) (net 14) (status 20))
 (segment (start 115.55001 32.77001) (end 114.95 32.17) (width 0.4) (layer F.Cu) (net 14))
 (segment (start 115.55001 35.170666) (end 115.55001 32.77001) (width 0.4) (layer F.Cu) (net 14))
 (segment (start 99.400001 60.199999) (end 99.400001 51.320675) (width 0.4) (layer F.Cu) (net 14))
 (segment (start 99.400001 51.320675) (end 115.55001 35.170666) (width 0.4) (layer F.Cu) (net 14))
 (segment (start 98 61.6) (end 99.400001 60.199999) (width 0.4) (layer F.Cu) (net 14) (status 10))
 (segment (start 96.46 33.125) (end 96.46 33.691384) (width 0.4) (layer F.Cu) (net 15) (status 30))
 (segment (start 96.46 35.1) (end 98.86 37.5) (width 0.4) (layer F.Cu) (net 15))
 (segment (start 96.46 33.125) (end 96.46 35.1) (width 0.4) (layer F.Cu) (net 15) (status 10))
 (segment (start 111.185 37.5) (end 113.975 34.71) (width 0.4) (layer F.Cu) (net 15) (status 20))
 (segment (start 98.86 37.5) (end 111.185 37.5) (width 0.4) (layer F.Cu) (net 15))
 (segment (start 110.249324 36.4) (end 113.209324 33.44) (width 0.4) (layer F.Cu) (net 16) (status 20))
 (segment (start 99.639989 35.511375) (end 100.528614 36.4) (width 0.4) (layer F.Cu) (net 16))
 (segment (start 99.639989 33.439989) (end 99.639989 35.511375) (width 0.4) (layer F.Cu) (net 16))
 (segment (start 113.209324 33.44) (end 113.975 33.44) (width 0.4) (layer F.Cu) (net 16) (status 30))
 (segment (start 99.325 33.125) (end 99.639989 33.439989) (width 0.4) (layer F.Cu) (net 16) (status 10))
 (segment (start 100.528614 36.4) (end 110.249324 36.4) (width 0.4) (layer F.Cu) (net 16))
 (segment (start 99 33.125) (end 99.325 33.125) (width 0.4) (layer F.Cu) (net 16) (status 30))
 (segment (start 99 28.075) (end 99 28.8) (width 0.4) (layer F.Cu) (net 17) (status 30))
 (segment (start 108.434999 35.300001) (end 109.025 34.71) (width 0.4) (layer F.Cu) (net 17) (status 20))
 (segment (start 100.439999 35.180001) (end 100.559999 35.300001) (width 0.4) (layer F.Cu) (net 17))
 (segment (start 100.439999 29.514999) (end 100.439999 35.180001) (width 0.4) (layer F.Cu) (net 17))
 (segment (start 100.559999 35.300001) (end 108.434999 35.300001) (width 0.4) (layer F.Cu) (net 17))
 (segment (start 99 28.075) (end 100.439999 29.514999) (width 0.4) (layer F.Cu) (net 17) (status 10))
 (segment (start 110 30.9) (end 109.025 30.9) (width 0.4) (layer F.Cu) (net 18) (status 20))
 (segment (start 112.39999 28.50001) (end 110 30.9) (width 0.4) (layer F.Cu) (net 18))
 (segment (start 112.39999 23.05001) (end 112.39999 28.50001) (width 0.4) (layer F.Cu) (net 18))
 (segment (start 115.1 20.35) (end 112.39999 23.05001) (width 0.4) (layer F.Cu) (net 18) (status 10))
 (segment (start 103.765 30.9) (end 109.025 30.9) (width 0.4) (layer F.Cu) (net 18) (status 20))
 (segment (start 101.54 33.125) (end 103.765 30.9) (width 0.4) (layer F.Cu) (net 18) (status 10)))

